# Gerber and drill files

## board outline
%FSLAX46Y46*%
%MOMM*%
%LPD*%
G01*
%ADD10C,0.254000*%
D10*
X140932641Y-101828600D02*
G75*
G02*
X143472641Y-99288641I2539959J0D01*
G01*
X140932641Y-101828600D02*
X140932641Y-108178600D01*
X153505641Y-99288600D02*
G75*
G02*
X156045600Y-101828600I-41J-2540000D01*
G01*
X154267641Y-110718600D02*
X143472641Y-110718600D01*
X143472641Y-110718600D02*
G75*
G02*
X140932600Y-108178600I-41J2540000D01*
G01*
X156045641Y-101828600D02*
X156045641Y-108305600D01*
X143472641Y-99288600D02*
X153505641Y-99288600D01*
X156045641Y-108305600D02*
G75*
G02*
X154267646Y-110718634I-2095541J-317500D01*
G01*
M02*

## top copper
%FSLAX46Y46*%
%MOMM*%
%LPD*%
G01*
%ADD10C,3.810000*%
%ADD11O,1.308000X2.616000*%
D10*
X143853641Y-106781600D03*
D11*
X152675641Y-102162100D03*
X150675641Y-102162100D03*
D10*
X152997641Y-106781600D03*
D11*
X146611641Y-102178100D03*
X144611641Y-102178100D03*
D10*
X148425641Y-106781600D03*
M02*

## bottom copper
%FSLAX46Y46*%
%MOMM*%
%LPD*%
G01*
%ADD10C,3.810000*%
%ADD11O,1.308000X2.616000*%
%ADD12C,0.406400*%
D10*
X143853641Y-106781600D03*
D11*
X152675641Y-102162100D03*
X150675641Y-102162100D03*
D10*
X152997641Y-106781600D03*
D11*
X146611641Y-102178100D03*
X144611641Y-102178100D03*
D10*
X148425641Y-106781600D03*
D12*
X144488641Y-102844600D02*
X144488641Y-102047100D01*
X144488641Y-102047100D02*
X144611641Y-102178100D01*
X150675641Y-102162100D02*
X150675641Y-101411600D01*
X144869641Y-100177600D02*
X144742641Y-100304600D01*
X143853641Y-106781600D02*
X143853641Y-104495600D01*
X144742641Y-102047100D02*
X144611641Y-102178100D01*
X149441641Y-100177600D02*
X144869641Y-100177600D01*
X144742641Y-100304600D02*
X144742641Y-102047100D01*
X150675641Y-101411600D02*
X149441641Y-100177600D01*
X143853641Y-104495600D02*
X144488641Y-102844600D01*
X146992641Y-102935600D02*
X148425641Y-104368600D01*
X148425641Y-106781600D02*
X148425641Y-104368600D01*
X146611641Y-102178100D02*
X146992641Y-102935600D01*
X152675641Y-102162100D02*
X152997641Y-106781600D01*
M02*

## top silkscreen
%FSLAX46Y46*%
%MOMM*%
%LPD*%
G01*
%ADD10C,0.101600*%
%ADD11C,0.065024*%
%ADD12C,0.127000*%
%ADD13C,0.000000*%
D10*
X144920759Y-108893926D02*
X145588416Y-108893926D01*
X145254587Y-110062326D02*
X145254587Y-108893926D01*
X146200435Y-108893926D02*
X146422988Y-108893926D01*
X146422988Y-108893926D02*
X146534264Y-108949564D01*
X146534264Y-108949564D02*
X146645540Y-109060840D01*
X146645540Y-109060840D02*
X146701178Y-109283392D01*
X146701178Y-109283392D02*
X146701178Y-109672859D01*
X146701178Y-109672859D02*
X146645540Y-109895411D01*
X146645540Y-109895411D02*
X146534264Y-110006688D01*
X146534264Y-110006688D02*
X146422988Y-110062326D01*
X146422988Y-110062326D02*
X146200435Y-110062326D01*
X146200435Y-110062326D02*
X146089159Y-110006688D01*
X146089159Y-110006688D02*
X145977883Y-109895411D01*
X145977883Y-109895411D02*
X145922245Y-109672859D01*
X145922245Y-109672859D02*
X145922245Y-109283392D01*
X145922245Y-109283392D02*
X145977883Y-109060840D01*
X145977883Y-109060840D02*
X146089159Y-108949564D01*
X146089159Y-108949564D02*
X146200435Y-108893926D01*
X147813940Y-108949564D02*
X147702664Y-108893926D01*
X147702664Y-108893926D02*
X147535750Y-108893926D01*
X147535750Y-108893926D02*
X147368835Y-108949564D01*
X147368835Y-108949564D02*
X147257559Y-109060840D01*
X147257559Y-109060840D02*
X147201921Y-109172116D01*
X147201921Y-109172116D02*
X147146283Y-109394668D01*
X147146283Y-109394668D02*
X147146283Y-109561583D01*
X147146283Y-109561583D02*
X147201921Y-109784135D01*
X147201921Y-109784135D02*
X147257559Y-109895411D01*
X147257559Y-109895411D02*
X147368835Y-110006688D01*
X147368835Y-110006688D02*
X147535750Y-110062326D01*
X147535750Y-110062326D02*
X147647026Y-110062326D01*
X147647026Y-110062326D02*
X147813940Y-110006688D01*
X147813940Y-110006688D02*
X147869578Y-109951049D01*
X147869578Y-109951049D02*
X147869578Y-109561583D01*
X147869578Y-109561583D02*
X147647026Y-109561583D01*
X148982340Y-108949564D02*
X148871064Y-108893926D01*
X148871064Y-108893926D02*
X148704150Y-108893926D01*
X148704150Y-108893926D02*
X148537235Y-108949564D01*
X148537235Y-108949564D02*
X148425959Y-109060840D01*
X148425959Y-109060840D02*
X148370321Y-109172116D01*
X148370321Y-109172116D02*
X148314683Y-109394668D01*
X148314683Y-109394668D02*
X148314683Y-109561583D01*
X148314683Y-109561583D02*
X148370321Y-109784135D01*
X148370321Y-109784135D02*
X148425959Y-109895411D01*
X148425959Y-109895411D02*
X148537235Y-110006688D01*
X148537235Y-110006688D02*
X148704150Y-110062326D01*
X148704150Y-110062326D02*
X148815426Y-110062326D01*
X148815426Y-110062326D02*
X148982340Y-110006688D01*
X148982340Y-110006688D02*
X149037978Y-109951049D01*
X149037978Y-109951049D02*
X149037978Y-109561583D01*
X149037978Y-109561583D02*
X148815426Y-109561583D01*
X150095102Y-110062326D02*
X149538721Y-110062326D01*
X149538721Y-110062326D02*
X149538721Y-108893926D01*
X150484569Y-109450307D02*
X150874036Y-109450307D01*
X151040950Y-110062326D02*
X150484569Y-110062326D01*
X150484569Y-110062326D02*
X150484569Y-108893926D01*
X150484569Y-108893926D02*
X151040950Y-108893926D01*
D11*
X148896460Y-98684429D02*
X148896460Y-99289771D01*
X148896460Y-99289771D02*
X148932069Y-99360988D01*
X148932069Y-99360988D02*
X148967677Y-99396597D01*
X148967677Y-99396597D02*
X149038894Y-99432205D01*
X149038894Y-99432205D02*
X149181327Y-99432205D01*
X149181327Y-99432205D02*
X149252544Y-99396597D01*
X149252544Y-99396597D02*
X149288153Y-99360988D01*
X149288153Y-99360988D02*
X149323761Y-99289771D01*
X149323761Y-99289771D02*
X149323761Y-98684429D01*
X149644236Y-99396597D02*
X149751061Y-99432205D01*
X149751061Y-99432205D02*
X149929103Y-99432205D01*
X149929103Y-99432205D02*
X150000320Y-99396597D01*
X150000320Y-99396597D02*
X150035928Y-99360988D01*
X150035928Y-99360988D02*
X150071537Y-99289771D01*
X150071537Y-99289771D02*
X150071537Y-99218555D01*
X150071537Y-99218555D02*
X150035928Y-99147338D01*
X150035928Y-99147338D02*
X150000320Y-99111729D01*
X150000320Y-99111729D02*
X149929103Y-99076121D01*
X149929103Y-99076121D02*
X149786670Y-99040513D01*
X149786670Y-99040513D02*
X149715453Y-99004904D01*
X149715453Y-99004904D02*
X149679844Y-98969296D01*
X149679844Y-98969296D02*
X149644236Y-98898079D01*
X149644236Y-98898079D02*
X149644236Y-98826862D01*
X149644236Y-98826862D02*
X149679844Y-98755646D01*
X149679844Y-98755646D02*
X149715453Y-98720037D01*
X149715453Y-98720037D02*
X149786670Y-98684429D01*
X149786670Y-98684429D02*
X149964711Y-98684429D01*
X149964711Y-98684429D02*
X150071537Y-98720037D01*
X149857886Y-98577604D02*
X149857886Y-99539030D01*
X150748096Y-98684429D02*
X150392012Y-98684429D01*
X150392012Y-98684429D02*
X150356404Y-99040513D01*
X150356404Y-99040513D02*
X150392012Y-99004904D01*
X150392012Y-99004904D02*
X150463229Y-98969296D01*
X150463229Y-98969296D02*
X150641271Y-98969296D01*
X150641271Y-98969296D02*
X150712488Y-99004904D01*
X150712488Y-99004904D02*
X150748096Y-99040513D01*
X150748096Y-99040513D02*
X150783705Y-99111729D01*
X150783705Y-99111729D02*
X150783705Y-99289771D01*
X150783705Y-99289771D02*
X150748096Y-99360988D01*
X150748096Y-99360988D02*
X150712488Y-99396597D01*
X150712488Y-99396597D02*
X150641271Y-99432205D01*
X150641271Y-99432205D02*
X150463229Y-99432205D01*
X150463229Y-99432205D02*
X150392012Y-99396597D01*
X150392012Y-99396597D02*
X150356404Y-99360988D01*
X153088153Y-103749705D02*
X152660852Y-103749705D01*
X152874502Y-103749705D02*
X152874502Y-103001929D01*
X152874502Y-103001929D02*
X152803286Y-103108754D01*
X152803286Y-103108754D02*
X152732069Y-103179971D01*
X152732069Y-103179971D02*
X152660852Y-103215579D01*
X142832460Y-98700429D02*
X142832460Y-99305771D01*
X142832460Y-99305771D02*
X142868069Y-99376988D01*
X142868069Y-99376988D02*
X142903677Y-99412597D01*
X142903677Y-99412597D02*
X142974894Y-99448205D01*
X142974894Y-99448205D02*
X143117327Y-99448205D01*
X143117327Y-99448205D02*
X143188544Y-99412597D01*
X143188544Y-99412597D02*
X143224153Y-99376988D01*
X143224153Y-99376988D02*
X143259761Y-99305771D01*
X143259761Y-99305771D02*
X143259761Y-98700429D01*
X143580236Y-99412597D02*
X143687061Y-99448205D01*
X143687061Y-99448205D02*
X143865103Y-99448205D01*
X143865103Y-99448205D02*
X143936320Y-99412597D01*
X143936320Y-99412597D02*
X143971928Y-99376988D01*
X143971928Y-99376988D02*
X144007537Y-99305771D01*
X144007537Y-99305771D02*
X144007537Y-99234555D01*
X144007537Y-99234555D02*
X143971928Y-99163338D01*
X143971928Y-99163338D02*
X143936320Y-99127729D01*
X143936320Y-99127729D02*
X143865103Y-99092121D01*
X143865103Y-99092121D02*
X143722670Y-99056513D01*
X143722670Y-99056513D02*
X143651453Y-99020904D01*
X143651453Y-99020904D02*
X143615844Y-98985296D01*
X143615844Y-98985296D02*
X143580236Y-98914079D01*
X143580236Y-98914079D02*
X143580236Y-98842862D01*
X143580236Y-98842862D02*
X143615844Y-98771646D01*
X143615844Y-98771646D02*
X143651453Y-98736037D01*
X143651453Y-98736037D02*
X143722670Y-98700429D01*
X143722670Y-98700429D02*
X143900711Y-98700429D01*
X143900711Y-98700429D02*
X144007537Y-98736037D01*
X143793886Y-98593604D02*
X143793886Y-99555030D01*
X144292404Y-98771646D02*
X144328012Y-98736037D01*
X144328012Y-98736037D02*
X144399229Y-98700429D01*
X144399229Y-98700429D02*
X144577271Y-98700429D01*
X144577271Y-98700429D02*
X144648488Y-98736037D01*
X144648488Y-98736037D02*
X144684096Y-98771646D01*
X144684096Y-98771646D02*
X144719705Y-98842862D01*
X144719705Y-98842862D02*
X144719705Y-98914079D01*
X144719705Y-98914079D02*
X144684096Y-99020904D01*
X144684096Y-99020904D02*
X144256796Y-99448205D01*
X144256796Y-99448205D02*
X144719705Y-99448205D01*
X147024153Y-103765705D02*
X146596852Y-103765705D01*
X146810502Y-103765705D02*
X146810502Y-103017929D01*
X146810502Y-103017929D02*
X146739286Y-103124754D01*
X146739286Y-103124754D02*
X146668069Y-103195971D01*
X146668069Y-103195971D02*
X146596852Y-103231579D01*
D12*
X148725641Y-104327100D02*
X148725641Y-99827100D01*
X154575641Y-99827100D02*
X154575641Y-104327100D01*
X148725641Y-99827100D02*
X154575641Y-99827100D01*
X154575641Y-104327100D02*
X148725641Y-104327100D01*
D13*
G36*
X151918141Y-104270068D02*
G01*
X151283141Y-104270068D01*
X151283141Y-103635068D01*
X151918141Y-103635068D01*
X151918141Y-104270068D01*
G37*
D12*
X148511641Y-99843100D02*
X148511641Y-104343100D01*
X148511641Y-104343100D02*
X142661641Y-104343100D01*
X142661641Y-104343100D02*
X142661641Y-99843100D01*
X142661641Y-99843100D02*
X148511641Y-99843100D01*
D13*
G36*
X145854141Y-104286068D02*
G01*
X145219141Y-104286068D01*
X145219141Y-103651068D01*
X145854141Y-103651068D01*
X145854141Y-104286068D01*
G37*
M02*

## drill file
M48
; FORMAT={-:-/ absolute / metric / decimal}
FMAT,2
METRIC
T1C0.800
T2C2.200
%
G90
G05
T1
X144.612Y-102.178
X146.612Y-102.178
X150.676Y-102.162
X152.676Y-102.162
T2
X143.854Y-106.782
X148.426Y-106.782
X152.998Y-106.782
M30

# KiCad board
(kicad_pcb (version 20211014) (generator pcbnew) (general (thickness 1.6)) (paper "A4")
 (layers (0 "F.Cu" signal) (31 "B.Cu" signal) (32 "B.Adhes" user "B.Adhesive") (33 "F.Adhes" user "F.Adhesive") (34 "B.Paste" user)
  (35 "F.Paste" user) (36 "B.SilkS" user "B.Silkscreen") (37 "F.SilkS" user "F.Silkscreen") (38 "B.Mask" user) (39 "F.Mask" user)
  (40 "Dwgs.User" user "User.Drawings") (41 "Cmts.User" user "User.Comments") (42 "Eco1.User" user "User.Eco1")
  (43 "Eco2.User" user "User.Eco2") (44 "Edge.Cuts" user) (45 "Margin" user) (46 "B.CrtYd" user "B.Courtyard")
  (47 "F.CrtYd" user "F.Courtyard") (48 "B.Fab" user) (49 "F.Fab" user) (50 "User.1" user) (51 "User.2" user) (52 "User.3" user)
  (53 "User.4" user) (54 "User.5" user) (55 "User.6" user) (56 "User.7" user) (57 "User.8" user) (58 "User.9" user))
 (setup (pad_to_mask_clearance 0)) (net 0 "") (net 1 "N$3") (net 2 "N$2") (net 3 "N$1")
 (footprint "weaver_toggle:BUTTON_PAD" (layer "F.Cu") (at 143.853641 106.7816)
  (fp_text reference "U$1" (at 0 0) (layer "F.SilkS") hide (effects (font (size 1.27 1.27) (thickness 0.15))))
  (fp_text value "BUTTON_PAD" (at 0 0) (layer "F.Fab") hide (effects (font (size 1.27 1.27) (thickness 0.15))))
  (pad "P$1" thru_hole circle (at 0 0) (size 3.81 3.81) (drill 2.2) (layers *.Cu *.Mask) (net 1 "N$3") (solder_mask_margin 0.1016)))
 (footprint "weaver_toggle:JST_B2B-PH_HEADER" (layer "F.Cu") (at 151.600641 102.2096)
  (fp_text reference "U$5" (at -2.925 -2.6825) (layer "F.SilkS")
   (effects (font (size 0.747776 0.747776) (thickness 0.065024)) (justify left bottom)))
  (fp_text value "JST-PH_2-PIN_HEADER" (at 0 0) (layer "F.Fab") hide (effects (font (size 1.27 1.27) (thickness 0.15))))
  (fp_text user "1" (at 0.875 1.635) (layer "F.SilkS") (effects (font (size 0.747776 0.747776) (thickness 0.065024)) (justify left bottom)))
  (fp_line (start -2.875 2.1175) (end -2.875 -2.3825) (layer "F.SilkS") (width 0.127))
  (fp_line (start 2.975 -2.3825) (end 2.975 2.1175) (layer "F.SilkS") (width 0.127))
  (fp_line (start -2.875 -2.3825) (end 2.975 -2.3825) (layer "F.SilkS") (width 0.127))
  (fp_line (start 2.975 2.1175) (end -2.875 2.1175) (layer "F.SilkS") (width 0.127))
  (fp_poly
   (pts (xy -0.3175 2.060468) (xy 0.3175 2.060468) (xy 0.3175 1.425468) (xy -0.3175 1.425468)) (layer "F.SilkS") (width 0) (fill solid))
  (pad "P1" thru_hole oval (at 1.075 -0.0475 90) (size 2.616 1.308) (drill 0.8) (layers *.Cu *.Mask) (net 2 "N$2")
   (solder_mask_margin 0.1016))
  (pad "P2" thru_hole oval (at -0.925 -0.0475 90) (size 2.616 1.308) (drill 0.8) (layers *.Cu *.Mask) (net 1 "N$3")
   (solder_mask_margin 0.1016)))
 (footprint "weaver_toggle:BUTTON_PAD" (layer "F.Cu") (at 152.997641 106.7816)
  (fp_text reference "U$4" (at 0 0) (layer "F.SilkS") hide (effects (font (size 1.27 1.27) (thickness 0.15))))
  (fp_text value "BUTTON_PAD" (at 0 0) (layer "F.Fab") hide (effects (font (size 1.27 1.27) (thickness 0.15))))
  (pad "P$1" thru_hole circle (at 0 0) (size 3.81 3.81) (drill 2.2) (layers *.Cu *.Mask) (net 2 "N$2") (solder_mask_margin 0.1016)))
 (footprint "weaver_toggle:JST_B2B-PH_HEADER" (layer "F.Cu") (at 145.536641 102.2256)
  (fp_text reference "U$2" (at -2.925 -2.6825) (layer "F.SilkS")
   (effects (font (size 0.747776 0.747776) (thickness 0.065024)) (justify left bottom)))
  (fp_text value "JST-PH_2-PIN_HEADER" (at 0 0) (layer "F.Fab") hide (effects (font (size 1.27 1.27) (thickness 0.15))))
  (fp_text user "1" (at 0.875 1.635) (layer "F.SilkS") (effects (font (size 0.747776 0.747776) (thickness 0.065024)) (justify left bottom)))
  (fp_line (start 2.975 -2.3825) (end 2.975 2.1175) (layer "F.SilkS") (width 0.127))
  (fp_line (start 2.975 2.1175) (end -2.875 2.1175) (layer "F.SilkS") (width 0.127))
  (fp_line (start -2.875 2.1175) (end -2.875 -2.3825) (layer "F.SilkS") (width 0.127))
  (fp_line (start -2.875 -2.3825) (end 2.975 -2.3825) (layer "F.SilkS") (width 0.127))
  (fp_poly
   (pts (xy -0.3175 2.060468) (xy 0.3175 2.060468) (xy 0.3175 1.425468) (xy -0.3175 1.425468)) (layer "F.SilkS") (width 0) (fill solid))
  (pad "P1" thru_hole oval (at 1.075 -0.0475 90) (size 2.616 1.308) (drill 0.8) (layers *.Cu *.Mask) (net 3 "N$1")
   (solder_mask_margin 0.1016))
  (pad "P2" thru_hole oval (at -0.925 -0.0475 90) (size 2.616 1.308) (drill 0.8) (layers *.Cu *.Mask) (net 1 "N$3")
   (solder_mask_margin 0.1016)))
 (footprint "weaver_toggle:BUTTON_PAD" (layer "F.Cu") (at 148.425641 106.7816)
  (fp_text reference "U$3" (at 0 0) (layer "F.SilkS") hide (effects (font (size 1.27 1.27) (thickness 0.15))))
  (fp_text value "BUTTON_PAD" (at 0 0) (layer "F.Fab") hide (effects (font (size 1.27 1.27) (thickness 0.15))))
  (pad "P$1" thru_hole circle (at 0 0) (size 3.81 3.81) (drill 2.2) (layers *.Cu *.Mask) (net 3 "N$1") (solder_mask_margin 0.1016)))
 (gr_arc (start 140.932641 101.8286) (mid 141.67659 100.032549) (end 143.472641 99.2886) (layer "Edge.Cuts") (width 0.254))
 (gr_line (start 140.932641 101.8286) (end 140.932641 108.1786) (layer "Edge.Cuts") (width 0.254))
 (gr_arc (start 153.505641 99.2886) (mid 155.301692 100.032549) (end 156.045641 101.8286) (layer "Edge.Cuts") (width 0.254))
 (gr_line (start 154.267641 110.7186) (end 143.472641 110.7186) (layer "Edge.Cuts") (width 0.254))
 (gr_arc (start 143.472641 110.7186) (mid 141.67659 109.974651) (end 140.932641 108.1786) (layer "Edge.Cuts") (width 0.254))
 (gr_line (start 156.045641 101.8286) (end 156.045641 108.3056) (layer "Edge.Cuts") (width 0.254))
 (gr_line (start 143.472641 99.2886) (end 153.505641 99.2886) (layer "Edge.Cuts") (width 0.254))
 (gr_arc (start 156.045641 108.3056) (mid 155.65639 109.880336) (end 154.267641 110.7186) (layer "Edge.Cuts") (width 0.254))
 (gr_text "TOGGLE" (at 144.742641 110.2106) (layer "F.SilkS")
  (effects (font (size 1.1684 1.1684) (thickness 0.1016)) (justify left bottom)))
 (segment (start 144.488641 102.8446) (end 144.488641 102.0471) (width 0.4064) (layer "B.Cu") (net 1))
 (segment (start 144.488641 102.0471) (end 144.611641 102.1781) (width 0.4064) (layer "B.Cu") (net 1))
 (segment (start 150.675641 102.1621) (end 150.675641 101.4116) (width 0.4064) (layer "B.Cu") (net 1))
 (segment (start 144.869641 100.1776) (end 144.742641 100.3046) (width 0.4064) (layer "B.Cu") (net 1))
 (segment (start 143.853641 106.7816) (end 143.853641 104.4956) (width 0.4064) (layer "B.Cu") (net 1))
 (segment (start 144.742641 102.0471) (end 144.611641 102.1781) (width 0.4064) (layer "B.Cu") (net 1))
 (segment (start 149.441641 100.1776) (end 144.869641 100.1776) (width 0.4064) (layer "B.Cu") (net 1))
 (segment (start 144.742641 100.3046) (end 144.742641 102.0471) (width 0.4064) (layer "B.Cu") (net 1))
 (segment (start 150.675641 101.4116) (end 149.441641 100.1776) (width 0.4064) (layer "B.Cu") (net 1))
 (segment (start 143.853641 104.4956) (end 144.488641 102.8446) (width 0.4064) (layer "B.Cu") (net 1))
 (segment (start 146.992641 102.9356) (end 148.425641 104.3686) (width 0.4064) (layer "B.Cu") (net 3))
 (segment (start 148.425641 106.7816) (end 148.425641 104.3686) (width 0.4064) (layer "B.Cu") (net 3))
 (segment (start 146.611641 102.1781) (end 146.992641 102.9356) (width 0.4064) (layer "B.Cu") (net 3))
 (segment (start 152.675641 102.1621) (end 152.997641 106.7816) (width 0.4064) (layer "B.Cu") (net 2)))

